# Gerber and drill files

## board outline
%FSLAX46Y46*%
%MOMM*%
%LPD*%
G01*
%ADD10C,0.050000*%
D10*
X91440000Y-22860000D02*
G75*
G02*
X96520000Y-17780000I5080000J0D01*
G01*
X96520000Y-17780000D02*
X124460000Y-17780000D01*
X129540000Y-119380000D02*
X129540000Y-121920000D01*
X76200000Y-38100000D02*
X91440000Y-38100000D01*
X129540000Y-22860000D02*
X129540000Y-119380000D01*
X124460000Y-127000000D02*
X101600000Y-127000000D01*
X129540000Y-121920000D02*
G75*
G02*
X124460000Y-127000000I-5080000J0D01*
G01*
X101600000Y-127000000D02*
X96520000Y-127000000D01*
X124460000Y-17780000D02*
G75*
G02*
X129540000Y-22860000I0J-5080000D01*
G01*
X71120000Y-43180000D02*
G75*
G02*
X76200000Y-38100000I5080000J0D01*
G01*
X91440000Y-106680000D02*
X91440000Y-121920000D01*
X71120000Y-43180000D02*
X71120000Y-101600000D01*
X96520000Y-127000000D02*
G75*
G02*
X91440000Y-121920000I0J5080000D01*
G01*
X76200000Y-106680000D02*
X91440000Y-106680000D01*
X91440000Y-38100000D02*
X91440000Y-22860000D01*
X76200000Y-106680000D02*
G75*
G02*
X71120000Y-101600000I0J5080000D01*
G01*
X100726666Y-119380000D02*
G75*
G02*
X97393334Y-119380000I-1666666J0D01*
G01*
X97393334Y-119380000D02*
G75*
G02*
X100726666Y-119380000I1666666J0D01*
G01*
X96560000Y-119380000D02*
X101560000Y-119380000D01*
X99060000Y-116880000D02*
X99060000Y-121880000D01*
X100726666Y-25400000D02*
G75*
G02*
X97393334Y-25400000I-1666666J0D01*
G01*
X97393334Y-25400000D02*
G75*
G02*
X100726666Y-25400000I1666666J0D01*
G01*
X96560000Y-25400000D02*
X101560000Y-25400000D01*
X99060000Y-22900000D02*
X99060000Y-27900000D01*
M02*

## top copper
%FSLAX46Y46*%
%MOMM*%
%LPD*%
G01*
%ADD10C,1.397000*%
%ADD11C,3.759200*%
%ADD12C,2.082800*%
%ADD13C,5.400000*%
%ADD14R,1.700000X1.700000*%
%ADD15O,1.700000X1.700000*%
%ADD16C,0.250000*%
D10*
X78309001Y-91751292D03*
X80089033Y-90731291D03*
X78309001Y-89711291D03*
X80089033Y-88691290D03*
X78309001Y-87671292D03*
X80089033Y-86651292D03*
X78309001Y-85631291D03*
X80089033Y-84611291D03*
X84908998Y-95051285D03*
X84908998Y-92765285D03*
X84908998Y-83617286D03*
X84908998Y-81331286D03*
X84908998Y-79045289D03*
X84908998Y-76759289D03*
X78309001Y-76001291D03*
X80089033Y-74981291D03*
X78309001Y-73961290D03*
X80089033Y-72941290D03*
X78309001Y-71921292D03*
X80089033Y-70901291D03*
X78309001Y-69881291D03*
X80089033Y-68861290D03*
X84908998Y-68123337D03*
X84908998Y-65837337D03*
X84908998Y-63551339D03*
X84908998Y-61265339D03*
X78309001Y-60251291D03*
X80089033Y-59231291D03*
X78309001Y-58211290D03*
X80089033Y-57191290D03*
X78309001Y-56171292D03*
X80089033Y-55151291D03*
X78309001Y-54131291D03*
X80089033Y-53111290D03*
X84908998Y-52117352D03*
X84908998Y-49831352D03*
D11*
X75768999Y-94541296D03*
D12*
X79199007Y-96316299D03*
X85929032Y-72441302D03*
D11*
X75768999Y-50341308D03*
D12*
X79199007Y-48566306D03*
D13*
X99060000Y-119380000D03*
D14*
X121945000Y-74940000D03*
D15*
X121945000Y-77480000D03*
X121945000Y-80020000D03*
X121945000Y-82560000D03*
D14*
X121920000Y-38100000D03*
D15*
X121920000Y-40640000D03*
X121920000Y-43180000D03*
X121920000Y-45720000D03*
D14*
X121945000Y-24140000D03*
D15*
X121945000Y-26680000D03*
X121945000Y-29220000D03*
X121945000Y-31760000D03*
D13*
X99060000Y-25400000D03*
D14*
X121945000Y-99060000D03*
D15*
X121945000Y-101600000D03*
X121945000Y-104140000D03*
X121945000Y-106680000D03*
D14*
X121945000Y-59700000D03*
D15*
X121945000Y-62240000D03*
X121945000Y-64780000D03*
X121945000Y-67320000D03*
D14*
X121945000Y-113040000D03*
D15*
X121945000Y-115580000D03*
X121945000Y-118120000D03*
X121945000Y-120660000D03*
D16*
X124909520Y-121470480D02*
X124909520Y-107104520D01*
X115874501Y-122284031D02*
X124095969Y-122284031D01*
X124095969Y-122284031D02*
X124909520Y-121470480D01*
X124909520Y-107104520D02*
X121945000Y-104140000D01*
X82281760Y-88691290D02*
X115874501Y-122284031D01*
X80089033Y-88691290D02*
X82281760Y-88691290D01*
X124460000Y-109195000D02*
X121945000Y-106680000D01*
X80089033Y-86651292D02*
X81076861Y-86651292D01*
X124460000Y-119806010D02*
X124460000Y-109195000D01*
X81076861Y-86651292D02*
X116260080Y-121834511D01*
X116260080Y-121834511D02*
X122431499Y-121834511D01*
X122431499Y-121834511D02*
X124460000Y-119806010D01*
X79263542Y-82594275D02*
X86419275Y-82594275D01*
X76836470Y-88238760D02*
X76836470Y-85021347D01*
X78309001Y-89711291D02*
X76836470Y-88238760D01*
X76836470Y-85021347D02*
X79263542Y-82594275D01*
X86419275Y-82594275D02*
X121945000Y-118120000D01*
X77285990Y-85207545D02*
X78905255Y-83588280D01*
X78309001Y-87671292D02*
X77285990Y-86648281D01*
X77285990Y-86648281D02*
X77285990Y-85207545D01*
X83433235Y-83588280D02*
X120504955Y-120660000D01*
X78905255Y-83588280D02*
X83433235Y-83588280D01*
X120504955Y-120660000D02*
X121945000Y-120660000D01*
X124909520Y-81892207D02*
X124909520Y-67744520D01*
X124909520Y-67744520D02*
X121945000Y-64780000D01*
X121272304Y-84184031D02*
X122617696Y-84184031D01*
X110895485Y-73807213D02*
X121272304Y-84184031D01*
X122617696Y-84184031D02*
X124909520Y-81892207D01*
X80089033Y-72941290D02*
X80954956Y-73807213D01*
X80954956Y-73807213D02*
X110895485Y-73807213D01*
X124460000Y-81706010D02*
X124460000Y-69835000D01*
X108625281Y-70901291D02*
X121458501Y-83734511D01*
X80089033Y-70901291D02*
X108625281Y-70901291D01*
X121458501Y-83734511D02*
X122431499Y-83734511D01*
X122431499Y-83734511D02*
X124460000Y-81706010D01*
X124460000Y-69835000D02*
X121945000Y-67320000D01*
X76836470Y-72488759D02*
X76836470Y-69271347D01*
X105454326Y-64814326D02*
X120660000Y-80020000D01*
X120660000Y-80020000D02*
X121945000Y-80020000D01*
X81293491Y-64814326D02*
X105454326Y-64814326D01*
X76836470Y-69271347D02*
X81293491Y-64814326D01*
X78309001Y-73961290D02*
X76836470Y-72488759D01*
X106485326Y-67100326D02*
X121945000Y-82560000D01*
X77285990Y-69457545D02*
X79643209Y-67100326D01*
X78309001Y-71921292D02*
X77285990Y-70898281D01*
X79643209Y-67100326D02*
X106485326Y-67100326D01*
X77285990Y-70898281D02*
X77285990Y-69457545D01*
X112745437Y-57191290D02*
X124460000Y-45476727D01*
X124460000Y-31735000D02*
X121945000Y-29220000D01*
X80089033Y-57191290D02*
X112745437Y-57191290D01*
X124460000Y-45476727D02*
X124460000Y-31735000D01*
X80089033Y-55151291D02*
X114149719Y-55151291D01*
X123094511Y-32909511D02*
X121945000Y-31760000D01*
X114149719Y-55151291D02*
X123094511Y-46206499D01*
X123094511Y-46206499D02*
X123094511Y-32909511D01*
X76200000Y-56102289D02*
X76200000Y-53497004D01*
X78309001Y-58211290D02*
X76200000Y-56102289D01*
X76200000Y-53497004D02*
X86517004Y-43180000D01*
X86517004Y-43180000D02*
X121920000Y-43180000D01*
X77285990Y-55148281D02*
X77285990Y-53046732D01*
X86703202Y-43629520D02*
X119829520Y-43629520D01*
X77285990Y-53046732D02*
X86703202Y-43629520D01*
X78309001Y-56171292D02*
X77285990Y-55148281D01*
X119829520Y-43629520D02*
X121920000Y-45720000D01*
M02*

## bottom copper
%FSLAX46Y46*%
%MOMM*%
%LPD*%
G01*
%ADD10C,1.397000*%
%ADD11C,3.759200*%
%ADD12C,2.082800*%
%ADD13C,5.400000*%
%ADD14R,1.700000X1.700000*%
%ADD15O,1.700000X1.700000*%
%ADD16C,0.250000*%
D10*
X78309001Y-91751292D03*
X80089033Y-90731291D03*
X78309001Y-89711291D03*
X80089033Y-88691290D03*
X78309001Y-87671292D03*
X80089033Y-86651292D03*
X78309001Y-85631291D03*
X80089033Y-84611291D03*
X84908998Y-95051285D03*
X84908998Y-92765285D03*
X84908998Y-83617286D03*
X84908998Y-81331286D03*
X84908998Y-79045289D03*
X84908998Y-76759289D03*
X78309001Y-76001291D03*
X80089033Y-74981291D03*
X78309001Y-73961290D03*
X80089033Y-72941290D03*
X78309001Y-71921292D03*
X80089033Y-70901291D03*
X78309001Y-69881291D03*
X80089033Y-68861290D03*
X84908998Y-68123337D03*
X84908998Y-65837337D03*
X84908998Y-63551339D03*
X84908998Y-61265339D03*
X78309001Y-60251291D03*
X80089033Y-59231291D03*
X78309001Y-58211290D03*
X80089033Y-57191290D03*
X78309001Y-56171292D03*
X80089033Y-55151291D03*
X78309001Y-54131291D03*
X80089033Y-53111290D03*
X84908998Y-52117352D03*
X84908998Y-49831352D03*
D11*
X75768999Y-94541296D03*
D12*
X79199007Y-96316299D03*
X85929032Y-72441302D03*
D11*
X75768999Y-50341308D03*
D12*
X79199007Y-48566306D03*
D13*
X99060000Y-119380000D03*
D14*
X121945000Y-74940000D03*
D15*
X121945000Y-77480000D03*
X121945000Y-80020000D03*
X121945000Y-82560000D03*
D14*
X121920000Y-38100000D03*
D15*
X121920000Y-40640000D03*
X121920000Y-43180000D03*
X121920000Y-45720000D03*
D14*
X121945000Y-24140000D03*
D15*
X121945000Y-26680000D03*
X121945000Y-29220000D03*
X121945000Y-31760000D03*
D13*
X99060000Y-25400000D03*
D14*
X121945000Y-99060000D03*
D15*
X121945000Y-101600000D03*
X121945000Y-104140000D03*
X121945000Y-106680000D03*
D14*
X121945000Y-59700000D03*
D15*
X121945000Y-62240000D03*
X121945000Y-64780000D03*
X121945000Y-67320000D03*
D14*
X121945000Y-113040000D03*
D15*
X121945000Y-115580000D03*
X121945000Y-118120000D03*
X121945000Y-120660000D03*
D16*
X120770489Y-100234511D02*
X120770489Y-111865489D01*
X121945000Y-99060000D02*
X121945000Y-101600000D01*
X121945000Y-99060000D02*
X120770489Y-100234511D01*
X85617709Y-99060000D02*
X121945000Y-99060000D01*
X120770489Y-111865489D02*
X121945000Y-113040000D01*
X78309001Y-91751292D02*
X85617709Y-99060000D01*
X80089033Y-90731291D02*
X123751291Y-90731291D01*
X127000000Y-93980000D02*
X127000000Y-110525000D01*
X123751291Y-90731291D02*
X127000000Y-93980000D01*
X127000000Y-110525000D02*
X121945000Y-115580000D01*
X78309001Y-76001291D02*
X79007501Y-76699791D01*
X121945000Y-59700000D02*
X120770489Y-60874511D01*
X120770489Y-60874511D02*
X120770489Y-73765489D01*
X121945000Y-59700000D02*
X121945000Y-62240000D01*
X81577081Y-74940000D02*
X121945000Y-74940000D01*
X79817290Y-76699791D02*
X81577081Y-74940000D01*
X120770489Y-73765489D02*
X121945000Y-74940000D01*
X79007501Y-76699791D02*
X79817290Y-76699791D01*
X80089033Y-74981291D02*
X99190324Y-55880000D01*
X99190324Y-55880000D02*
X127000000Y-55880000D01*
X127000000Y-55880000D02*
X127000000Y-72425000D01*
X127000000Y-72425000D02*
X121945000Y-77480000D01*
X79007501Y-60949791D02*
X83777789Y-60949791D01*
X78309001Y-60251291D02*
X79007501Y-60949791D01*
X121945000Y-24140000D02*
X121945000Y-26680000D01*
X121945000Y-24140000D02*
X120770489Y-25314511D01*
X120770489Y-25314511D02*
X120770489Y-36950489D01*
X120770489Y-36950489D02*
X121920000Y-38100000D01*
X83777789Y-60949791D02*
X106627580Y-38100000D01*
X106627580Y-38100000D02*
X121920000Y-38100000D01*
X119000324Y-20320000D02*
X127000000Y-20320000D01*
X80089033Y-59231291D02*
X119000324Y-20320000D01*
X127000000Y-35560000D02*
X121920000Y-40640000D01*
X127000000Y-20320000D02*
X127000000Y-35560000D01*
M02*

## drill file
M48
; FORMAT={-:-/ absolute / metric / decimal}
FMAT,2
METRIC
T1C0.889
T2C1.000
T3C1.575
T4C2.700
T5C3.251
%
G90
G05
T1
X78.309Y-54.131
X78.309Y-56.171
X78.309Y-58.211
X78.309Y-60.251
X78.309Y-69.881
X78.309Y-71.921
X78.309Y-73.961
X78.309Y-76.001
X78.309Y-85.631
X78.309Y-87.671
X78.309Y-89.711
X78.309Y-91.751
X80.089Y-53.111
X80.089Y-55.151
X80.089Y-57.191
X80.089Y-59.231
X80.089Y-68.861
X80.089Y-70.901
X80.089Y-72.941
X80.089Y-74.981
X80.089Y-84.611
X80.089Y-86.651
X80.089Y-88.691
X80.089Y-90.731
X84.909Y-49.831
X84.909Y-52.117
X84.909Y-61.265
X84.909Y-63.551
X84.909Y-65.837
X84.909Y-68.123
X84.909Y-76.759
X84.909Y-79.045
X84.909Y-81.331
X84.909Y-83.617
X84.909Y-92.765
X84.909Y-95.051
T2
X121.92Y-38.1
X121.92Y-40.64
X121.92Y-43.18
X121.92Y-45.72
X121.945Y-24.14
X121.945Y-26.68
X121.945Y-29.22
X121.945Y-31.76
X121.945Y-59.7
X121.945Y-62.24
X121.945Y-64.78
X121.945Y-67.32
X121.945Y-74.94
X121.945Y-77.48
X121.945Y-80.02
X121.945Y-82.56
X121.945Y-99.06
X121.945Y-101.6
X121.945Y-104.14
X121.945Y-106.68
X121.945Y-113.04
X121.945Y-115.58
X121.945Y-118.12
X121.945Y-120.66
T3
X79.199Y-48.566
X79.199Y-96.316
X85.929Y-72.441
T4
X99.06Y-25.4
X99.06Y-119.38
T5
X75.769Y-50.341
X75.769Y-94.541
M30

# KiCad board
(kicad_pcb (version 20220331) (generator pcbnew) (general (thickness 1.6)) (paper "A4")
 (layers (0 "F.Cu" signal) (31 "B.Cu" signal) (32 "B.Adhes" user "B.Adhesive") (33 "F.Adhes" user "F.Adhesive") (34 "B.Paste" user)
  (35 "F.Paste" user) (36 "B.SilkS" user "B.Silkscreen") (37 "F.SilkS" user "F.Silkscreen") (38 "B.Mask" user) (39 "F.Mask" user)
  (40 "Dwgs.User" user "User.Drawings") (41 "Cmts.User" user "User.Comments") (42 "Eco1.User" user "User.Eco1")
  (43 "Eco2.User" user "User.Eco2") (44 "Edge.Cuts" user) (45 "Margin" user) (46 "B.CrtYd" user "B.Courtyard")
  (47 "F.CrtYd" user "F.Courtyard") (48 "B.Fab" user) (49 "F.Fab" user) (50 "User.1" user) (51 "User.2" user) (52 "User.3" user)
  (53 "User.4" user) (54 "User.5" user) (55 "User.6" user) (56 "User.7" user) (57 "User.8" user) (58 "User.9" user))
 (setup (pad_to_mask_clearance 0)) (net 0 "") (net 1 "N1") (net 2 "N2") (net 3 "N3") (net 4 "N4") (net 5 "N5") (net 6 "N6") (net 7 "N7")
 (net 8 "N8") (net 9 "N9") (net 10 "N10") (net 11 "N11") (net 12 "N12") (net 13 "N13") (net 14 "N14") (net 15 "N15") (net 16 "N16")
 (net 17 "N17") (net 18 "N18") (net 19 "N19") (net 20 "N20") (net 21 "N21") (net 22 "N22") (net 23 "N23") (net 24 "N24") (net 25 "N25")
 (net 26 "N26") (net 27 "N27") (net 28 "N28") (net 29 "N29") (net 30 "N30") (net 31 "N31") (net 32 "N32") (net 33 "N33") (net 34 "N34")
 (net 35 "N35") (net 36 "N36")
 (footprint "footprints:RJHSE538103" (layer "F.Cu") (at 78.309001 91.751291 90)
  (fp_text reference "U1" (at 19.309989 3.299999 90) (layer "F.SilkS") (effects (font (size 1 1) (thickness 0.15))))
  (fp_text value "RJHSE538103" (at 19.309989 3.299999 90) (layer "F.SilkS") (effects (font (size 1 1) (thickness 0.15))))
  (pad "1" thru_hole circle locked (at -0.000001 0 90) (size 1.397 1.397) (drill 0.889) (layers *.Cu *.Mask) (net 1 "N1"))
  (pad "2" thru_hole circle locked (at 1.02 1.780032 90) (size 1.397 1.397) (drill 0.889) (layers *.Cu *.Mask) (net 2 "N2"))
  (pad "3" thru_hole circle locked (at 2.04 0 90) (size 1.397 1.397) (drill 0.889) (layers *.Cu *.Mask) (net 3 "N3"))
  (pad "4" thru_hole circle locked (at 3.060001 1.780032 90) (size 1.397 1.397) (drill 0.889) (layers *.Cu *.Mask) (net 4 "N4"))
  (pad "5" thru_hole circle locked (at 4.079999 0 90) (size 1.397 1.397) (drill 0.889) (layers *.Cu *.Mask) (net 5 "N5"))
  (pad "6" thru_hole circle locked (at 5.099999 1.780032 90) (size 1.397 1.397) (drill 0.889) (layers *.Cu *.Mask) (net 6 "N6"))
  (pad "7" thru_hole circle locked (at 6.12 0 90) (size 1.397 1.397) (drill 0.889) (layers *.Cu *.Mask) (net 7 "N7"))
  (pad "8" thru_hole circle locked (at 7.14 1.780032 90) (size 1.397 1.397) (drill 0.889) (layers *.Cu *.Mask) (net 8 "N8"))
  (pad "9" thru_hole circle locked (at -3.299994 6.599997 90) (size 1.397 1.397) (drill 0.889) (layers *.Cu *.Mask) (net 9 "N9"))
  (pad "10" thru_hole circle locked (at -1.013994 6.599997 90) (size 1.397 1.397) (drill 0.889) (layers *.Cu *.Mask) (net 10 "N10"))
  (pad "11" thru_hole circle locked (at 8.134005 6.599997 90) (size 1.397 1.397) (drill 0.889) (layers *.Cu *.Mask) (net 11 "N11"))
  (pad "12" thru_hole circle locked (at 10.420005 6.599997 90) (size 1.397 1.397) (drill 0.889) (layers *.Cu *.Mask) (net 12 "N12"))
  (pad "13" thru_hole circle locked (at 12.706002 6.599997 90) (size 1.397 1.397) (drill 0.889) (layers *.Cu *.Mask) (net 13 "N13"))
  (pad "14" thru_hole circle locked (at 14.992002 6.599997 90) (size 1.397 1.397) (drill 0.889) (layers *.Cu *.Mask) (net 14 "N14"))
  (pad "15" thru_hole circle locked (at 15.75 0 90) (size 1.397 1.397) (drill 0.889) (layers *.Cu *.Mask) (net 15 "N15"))
  (pad "16" thru_hole circle locked (at 16.77 1.780032 90) (size 1.397 1.397) (drill 0.889) (layers *.Cu *.Mask) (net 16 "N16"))
  (pad "17" thru_hole circle locked (at 17.790001 0 90) (size 1.397 1.397) (drill 0.889) (layers *.Cu *.Mask) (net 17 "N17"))
  (pad "18" thru_hole circle locked (at 18.810001 1.780032 90) (size 1.397 1.397) (drill 0.889) (layers *.Cu *.Mask) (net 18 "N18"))
  (pad "19" thru_hole circle locked (at 19.829999 0 90) (size 1.397 1.397) (drill 0.889) (layers *.Cu *.Mask) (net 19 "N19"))
  (pad "20" thru_hole circle locked (at 20.85 1.780032 90) (size 1.397 1.397) (drill 0.889) (layers *.Cu *.Mask) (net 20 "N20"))
  (pad "21" thru_hole circle locked (at 21.87 0 90) (size 1.397 1.397) (drill 0.889) (layers *.Cu *.Mask) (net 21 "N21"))
  (pad "22" thru_hole circle locked (at 22.890001 1.780032 90) (size 1.397 1.397) (drill 0.889) (layers *.Cu *.Mask) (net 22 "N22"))
  (pad "23" thru_hole circle locked (at 23.627954 6.599997 90) (size 1.397 1.397) (drill 0.889) (layers *.Cu *.Mask) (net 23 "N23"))
  (pad "24" thru_hole circle locked (at 25.913954 6.599997 90) (size 1.397 1.397) (drill 0.889) (layers *.Cu *.Mask) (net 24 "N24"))
  (pad "25" thru_hole circle locked (at 28.199952 6.599997 90) (size 1.397 1.397) (drill 0.889) (layers *.Cu *.Mask) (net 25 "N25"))
  (pad "26" thru_hole circle locked (at 30.485952 6.599997 90) (size 1.397 1.397) (drill 0.889) (layers *.Cu *.Mask) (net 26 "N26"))
  (pad "27" thru_hole circle locked (at 31.5 0 90) (size 1.397 1.397) (drill 0.889) (layers *.Cu *.Mask) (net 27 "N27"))
  (pad "28" thru_hole circle locked (at 32.52 1.780032 90) (size 1.397 1.397) (drill 0.889) (layers *.Cu *.Mask) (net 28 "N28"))
  (pad "29" thru_hole circle locked (at 33.540001 0 90) (size 1.397 1.397) (drill 0.889) (layers *.Cu *.Mask) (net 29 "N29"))
  (pad "30" thru_hole circle locked (at 34.560001 1.780032 90) (size 1.397 1.397) (drill 0.889) (layers *.Cu *.Mask) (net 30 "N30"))
  (pad "31" thru_hole circle locked (at 35.579999 0 90) (size 1.397 1.397) (drill 0.889) (layers *.Cu *.Mask) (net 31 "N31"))
  (pad "32" thru_hole circle locked (at 36.6 1.780032 90) (size 1.397 1.397) (drill 0.889) (layers *.Cu *.Mask) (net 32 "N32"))
  (pad "33" thru_hole circle locked (at 37.62 0 90) (size 1.397 1.397) (drill 0.889) (layers *.Cu *.Mask) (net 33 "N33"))
  (pad "34" thru_hole circle locked (at 38.640001 1.780032 90) (size 1.397 1.397) (drill 0.889) (layers *.Cu *.Mask) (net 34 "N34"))
  (pad "35" thru_hole circle locked (at 39.633939 6.599997 90) (size 1.397 1.397) (drill 0.889) (layers *.Cu *.Mask) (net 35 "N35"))
  (pad "36" thru_hole circle locked (at 41.919939 6.599997 90) (size 1.397 1.397) (drill 0.889) (layers *.Cu *.Mask) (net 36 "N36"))
  (pad "37" thru_hole circle locked (at -2.790005 -2.540002 90) (size 3.7592 3.7592) (drill 3.2512) (layers *.Cu *.Mask))
  (pad "38" thru_hole circle locked (at -4.565008 0.890006 90) (size 2.0828 2.0828) (drill 1.5748) (layers *.Cu *.Mask))
  (pad "39" thru_hole circle locked (at 19.309989 7.620031 90) (size 2.0828 2.0828) (drill 1.5748) (layers *.Cu *.Mask))
  (pad "40" thru_hole circle locked (at 41.409983 -2.540002 90) (size 3.7592 3.7592) (drill 3.2512) (layers *.Cu *.Mask))
  (pad "41" thru_hole circle locked (at 43.184985 0.890006 90) (size 2.0828 2.0828) (drill 1.5748) (layers *.Cu *.Mask)))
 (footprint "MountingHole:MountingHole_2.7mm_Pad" (layer "F.Cu") (at 99.06 119.38)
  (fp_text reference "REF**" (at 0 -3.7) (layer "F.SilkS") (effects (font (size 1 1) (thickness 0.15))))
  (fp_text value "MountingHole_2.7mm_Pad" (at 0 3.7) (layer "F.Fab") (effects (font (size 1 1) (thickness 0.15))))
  (pad "1" thru_hole circle (at 0 0) (size 5.4 5.4) (drill 2.7) (layers *.Cu *.Mask)))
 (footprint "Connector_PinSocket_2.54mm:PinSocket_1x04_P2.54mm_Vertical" (layer "F.Cu") (at 121.945 74.94)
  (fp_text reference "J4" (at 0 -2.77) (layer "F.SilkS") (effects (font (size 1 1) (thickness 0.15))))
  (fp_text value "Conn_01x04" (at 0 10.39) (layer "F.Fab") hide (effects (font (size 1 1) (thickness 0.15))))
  (pad "1" thru_hole rect (at 0 0) (size 1.7 1.7) (drill 1) (layers *.Cu *.Mask) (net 15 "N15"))
  (pad "2" thru_hole oval (at 0 2.54) (size 1.7 1.7) (drill 1) (layers *.Cu *.Mask) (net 16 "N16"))
  (pad "3" thru_hole oval (at 0 5.08) (size 1.7 1.7) (drill 1) (layers *.Cu *.Mask) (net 17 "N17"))
  (pad "4" thru_hole oval (at 0 7.62) (size 1.7 1.7) (drill 1) (layers *.Cu *.Mask) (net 19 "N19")))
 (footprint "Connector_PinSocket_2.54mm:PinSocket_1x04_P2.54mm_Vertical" (layer "F.Cu") (at 121.92 38.1)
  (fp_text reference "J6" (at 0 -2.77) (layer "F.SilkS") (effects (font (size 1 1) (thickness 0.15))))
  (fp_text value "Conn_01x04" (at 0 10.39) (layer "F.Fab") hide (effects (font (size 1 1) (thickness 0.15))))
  (pad "1" thru_hole rect (at 0 0) (size 1.7 1.7) (drill 1) (layers *.Cu *.Mask) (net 27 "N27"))
  (pad "2" thru_hole oval (at 0 2.54) (size 1.7 1.7) (drill 1) (layers *.Cu *.Mask) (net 28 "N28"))
  (pad "3" thru_hole oval (at 0 5.08) (size 1.7 1.7) (drill 1) (layers *.Cu *.Mask) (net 29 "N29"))
  (pad "4" thru_hole oval (at 0 7.62) (size 1.7 1.7) (drill 1) (layers *.Cu *.Mask) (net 31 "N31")))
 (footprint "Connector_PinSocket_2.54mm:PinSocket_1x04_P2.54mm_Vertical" (layer "F.Cu") (at 121.945 24.14)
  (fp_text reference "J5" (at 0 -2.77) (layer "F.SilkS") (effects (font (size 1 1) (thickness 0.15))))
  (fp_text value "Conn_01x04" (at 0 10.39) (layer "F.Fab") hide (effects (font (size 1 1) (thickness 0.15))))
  (pad "1" thru_hole rect (at 0 0) (size 1.7 1.7) (drill 1) (layers *.Cu *.Mask) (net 27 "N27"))
  (pad "2" thru_hole oval (at 0 2.54) (size 1.7 1.7) (drill 1) (layers *.Cu *.Mask) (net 27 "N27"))
  (pad "3" thru_hole oval (at 0 5.08) (size 1.7 1.7) (drill 1) (layers *.Cu *.Mask) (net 30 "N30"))
  (pad "4" thru_hole oval (at 0 7.62) (size 1.7 1.7) (drill 1) (layers *.Cu *.Mask) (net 32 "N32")))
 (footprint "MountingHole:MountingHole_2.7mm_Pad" (layer "F.Cu") (at 99.06 25.4)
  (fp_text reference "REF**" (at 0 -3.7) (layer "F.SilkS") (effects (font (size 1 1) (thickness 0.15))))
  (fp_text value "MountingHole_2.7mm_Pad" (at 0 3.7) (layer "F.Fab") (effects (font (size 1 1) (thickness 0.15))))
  (pad "1" thru_hole circle (at 0 0) (size 5.4 5.4) (drill 2.7) (layers *.Cu *.Mask)))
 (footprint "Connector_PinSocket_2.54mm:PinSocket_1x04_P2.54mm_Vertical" (layer "F.Cu") (at 121.945 99.06)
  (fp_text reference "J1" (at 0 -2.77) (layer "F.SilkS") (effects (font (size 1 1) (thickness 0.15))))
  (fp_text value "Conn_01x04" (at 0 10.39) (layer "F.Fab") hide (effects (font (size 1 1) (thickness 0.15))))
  (pad "1" thru_hole rect (at 0 0) (size 1.7 1.7) (drill 1) (layers *.Cu *.Mask) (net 1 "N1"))
  (pad "2" thru_hole oval (at 0 2.54) (size 1.7 1.7) (drill 1) (layers *.Cu *.Mask) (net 1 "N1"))
  (pad "3" thru_hole oval (at 0 5.08) (size 1.7 1.7) (drill 1) (layers *.Cu *.Mask) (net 4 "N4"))
  (pad "4" thru_hole oval (at 0 7.62) (size 1.7 1.7) (drill 1) (layers *.Cu *.Mask) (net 6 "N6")))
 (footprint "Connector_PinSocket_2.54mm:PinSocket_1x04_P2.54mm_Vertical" (layer "F.Cu") (at 121.945 59.7)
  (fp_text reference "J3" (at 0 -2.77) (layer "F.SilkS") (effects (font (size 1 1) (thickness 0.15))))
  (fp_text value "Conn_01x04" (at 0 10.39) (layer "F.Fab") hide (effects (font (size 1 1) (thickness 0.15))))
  (pad "1" thru_hole rect (at 0 0) (size 1.7 1.7) (drill 1) (layers *.Cu *.Mask) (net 15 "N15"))
  (pad "2" thru_hole oval (at 0 2.54) (size 1.7 1.7) (drill 1) (layers *.Cu *.Mask) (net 15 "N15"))
  (pad "3" thru_hole oval (at 0 5.08) (size 1.7 1.7) (drill 1) (layers *.Cu *.Mask) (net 18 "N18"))
  (pad "4" thru_hole oval (at 0 7.62) (size 1.7 1.7) (drill 1) (layers *.Cu *.Mask) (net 20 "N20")))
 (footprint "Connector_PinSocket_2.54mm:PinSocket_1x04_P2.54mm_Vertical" (layer "F.Cu") (at 121.945 113.04)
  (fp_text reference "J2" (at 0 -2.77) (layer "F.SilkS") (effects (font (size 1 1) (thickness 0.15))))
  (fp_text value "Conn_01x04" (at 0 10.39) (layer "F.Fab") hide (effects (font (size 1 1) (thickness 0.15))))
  (pad "1" thru_hole rect (at 0 0) (size 1.7 1.7) (drill 1) (layers *.Cu *.Mask) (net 1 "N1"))
  (pad "2" thru_hole oval (at 0 2.54) (size 1.7 1.7) (drill 1) (layers *.Cu *.Mask) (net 2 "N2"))
  (pad "3" thru_hole oval (at 0 5.08) (size 1.7 1.7) (drill 1) (layers *.Cu *.Mask) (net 3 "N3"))
  (pad "4" thru_hole oval (at 0 7.62) (size 1.7 1.7) (drill 1) (layers *.Cu *.Mask) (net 5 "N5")))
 (gr_arc (start 91.44 22.86) (mid 92.927898 19.267898) (end 96.52 17.78) (stroke (width 0.05) (type default)) (layer "Edge.Cuts"))
 (gr_line (start 96.52 17.78) (end 124.46 17.78) (stroke (width 0.05) (type default)) (layer "Edge.Cuts"))
 (gr_line (start 129.54 119.38) (end 129.54 121.92) (stroke (width 0.05) (type default)) (layer "Edge.Cuts"))
 (gr_line (start 76.2 38.1) (end 91.44 38.1) (stroke (width 0.05) (type default)) (layer "Edge.Cuts"))
 (gr_line (start 129.54 22.86) (end 129.54 119.38) (stroke (width 0.05) (type default)) (layer "Edge.Cuts"))
 (gr_line (start 124.46 127) (end 101.6 127) (stroke (width 0.05) (type default)) (layer "Edge.Cuts"))
 (gr_arc (start 129.54 121.92) (mid 128.052102 125.512102) (end 124.46 127) (stroke (width 0.05) (type default)) (layer "Edge.Cuts"))
 (gr_line (start 101.6 127) (end 96.52 127) (stroke (width 0.05) (type default)) (layer "Edge.Cuts"))
 (gr_arc (start 124.46 17.78) (mid 128.052102 19.267898) (end 129.54 22.86) (stroke (width 0.05) (type default)) (layer "Edge.Cuts"))
 (gr_arc (start 71.12 43.18) (mid 72.607898 39.587898) (end 76.2 38.1) (stroke (width 0.05) (type default)) (layer "Edge.Cuts"))
 (gr_line (start 91.44 106.68) (end 91.44 121.92) (stroke (width 0.05) (type default)) (layer "Edge.Cuts"))
 (gr_line (start 71.12 43.18) (end 71.12 101.6) (stroke (width 0.05) (type default)) (layer "Edge.Cuts"))
 (gr_arc (start 96.52 127) (mid 92.927898 125.512102) (end 91.44 121.92) (stroke (width 0.05) (type default)) (layer "Edge.Cuts"))
 (gr_line (start 76.2 106.68) (end 91.44 106.68) (stroke (width 0.05) (type default)) (layer "Edge.Cuts"))
 (gr_line (start 91.44 38.1) (end 91.44 22.86) (stroke (width 0.05) (type default)) (layer "Edge.Cuts"))
 (gr_arc (start 76.2 106.68) (mid 72.607898 105.192102) (end 71.12 101.6) (stroke (width 0.05) (type default)) (layer "Edge.Cuts"))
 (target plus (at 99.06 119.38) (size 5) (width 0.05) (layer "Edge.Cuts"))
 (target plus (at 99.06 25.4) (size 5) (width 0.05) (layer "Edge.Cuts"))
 (segment (start 120.770489 100.234511) (end 120.770489 111.865489) (width 0.25) (layer "B.Cu") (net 1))
 (segment (start 121.945 99.06) (end 121.945 101.6) (width 0.25) (layer "B.Cu") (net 1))
 (segment (start 121.945 99.06) (end 120.770489 100.234511) (width 0.25) (layer "B.Cu") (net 1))
 (segment (start 85.617709 99.06) (end 121.945 99.06) (width 0.25) (layer "B.Cu") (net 1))
 (segment (start 120.770489 111.865489) (end 121.945 113.04) (width 0.25) (layer "B.Cu") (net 1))
 (segment (start 78.309001 91.751292) (end 85.617709 99.06) (width 0.25) (layer "B.Cu") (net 1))
 (segment (start 124.90952 121.47048) (end 124.90952 107.10452) (width 0.25) (layer "F.Cu") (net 4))
 (segment (start 115.874501 122.284031) (end 124.095969 122.284031) (width 0.25) (layer "F.Cu") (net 4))
 (segment (start 124.095969 122.284031) (end 124.90952 121.47048) (width 0.25) (layer "F.Cu") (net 4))
 (segment (start 124.90952 107.10452) (end 121.945 104.14) (width 0.25) (layer "F.Cu") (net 4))
 (segment (start 82.28176 88.69129) (end 115.874501 122.284031) (width 0.25) (layer "F.Cu") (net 4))
 (segment (start 80.089033 88.69129) (end 82.28176 88.69129) (width 0.25) (layer "F.Cu") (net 4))
 (segment (start 124.46 109.195) (end 121.945 106.68) (width 0.25) (layer "F.Cu") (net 6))
 (segment (start 80.089033 86.651292) (end 81.076861 86.651292) (width 0.25) (layer "F.Cu") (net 6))
 (segment (start 124.46 119.80601) (end 124.46 109.195) (width 0.25) (layer "F.Cu") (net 6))
 (segment (start 81.076861 86.651292) (end 116.26008 121.834511) (width 0.25) (layer "F.Cu") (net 6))
 (segment (start 116.26008 121.834511) (end 122.431499 121.834511) (width 0.25) (layer "F.Cu") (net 6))
 (segment (start 122.431499 121.834511) (end 124.46 119.80601) (width 0.25) (layer "F.Cu") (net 6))
 (segment (start 80.089033 90.731291) (end 123.751291 90.731291) (width 0.25) (layer "B.Cu") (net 2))
 (segment (start 127 93.98) (end 127 110.525) (width 0.25) (layer "B.Cu") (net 2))
 (segment (start 123.751291 90.731291) (end 127 93.98) (width 0.25) (layer "B.Cu") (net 2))
 (segment (start 127 110.525) (end 121.945 115.58) (width 0.25) (layer "B.Cu") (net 2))
 (segment (start 79.263542 82.594275) (end 86.419275 82.594275) (width 0.25) (layer "F.Cu") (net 3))
 (segment (start 76.83647 88.23876) (end 76.83647 85.021347) (width 0.25) (layer "F.Cu") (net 3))
 (segment (start 78.309001 89.711291) (end 76.83647 88.23876) (width 0.25) (layer "F.Cu") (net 3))
 (segment (start 76.83647 85.021347) (end 79.263542 82.594275) (width 0.25) (layer "F.Cu") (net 3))
 (segment (start 86.419275 82.594275) (end 121.945 118.12) (width 0.25) (layer "F.Cu") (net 3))
 (segment (start 77.28599 85.207545) (end 78.905255 83.58828) (width 0.25) (layer "F.Cu") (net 5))
 (segment (start 78.309001 87.671292) (end 77.28599 86.648281) (width 0.25) (layer "F.Cu") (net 5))
 (segment (start 77.28599 86.648281) (end 77.28599 85.207545) (width 0.25) (layer "F.Cu") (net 5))
 (segment (start 83.433235 83.58828) (end 120.504955 120.66) (width 0.25) (layer "F.Cu") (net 5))
 (segment (start 78.905255 83.58828) (end 83.433235 83.58828) (width 0.25) (layer "F.Cu") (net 5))
 (segment (start 120.504955 120.66) (end 121.945 120.66) (width 0.25) (layer "F.Cu") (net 5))
 (segment (start 78.309001 76.001291) (end 79.007501 76.699791) (width 0.25) (layer "B.Cu") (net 15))
 (segment (start 121.945 59.7) (end 120.770489 60.874511) (width 0.25) (layer "B.Cu") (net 15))
 (segment (start 120.770489 60.874511) (end 120.770489 73.765489) (width 0.25) (layer "B.Cu") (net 15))
 (segment (start 121.945 59.7) (end 121.945 62.24) (width 0.25) (layer "B.Cu") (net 15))
 (segment (start 81.577081 74.94) (end 121.945 74.94) (width 0.25) (layer "B.Cu") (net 15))
 (segment (start 79.81729 76.699791) (end 81.577081 74.94) (width 0.25) (layer "B.Cu") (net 15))
 (segment (start 120.770489 73.765489) (end 121.945 74.94) (width 0.25) (layer "B.Cu") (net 15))
 (segment (start 79.007501 76.699791) (end 79.81729 76.699791) (width 0.25) (layer "B.Cu") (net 15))
 (segment (start 124.90952 81.892207) (end 124.90952 67.74452) (width 0.25) (layer "F.Cu") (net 18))
 (segment (start 124.90952 67.74452) (end 121.945 64.78) (width 0.25) (layer "F.Cu") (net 18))
 (segment (start 121.272304 84.184031) (end 122.617696 84.184031) (width 0.25) (layer "F.Cu") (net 18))
 (segment (start 110.895485 73.807213) (end 121.272304 84.184031) (width 0.25) (layer "F.Cu") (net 18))
 (segment (start 122.617696 84.184031) (end 124.90952 81.892207) (width 0.25) (layer "F.Cu") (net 18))
 (segment (start 80.089033 72.94129) (end 80.954956 73.807213) (width 0.25) (layer "F.Cu") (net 18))
 (segment (start 80.954956 73.807213) (end 110.895485 73.807213) (width 0.25) (layer "F.Cu") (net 18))
 (segment (start 124.46 81.70601) (end 124.46 69.835) (width 0.25) (layer "F.Cu") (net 20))
 (segment (start 108.625281 70.901291) (end 121.458501 83.734511) (width 0.25) (layer "F.Cu") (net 20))
 (segment (start 80.089033 70.901291) (end 108.625281 70.901291) (width 0.25) (layer "F.Cu") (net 20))
 (segment (start 121.458501 83.734511) (end 122.431499 83.734511) (width 0.25) (layer "F.Cu") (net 20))
 (segment (start 122.431499 83.734511) (end 124.46 81.70601) (width 0.25) (layer "F.Cu") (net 20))
 (segment (start 124.46 69.835) (end 121.945 67.32) (width 0.25) (layer "F.Cu") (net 20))
 (segment (start 80.089033 74.981291) (end 99.190324 55.88) (width 0.25) (layer "B.Cu") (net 16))
 (segment (start 99.190324 55.88) (end 127 55.88) (width 0.25) (layer "B.Cu") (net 16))
 (segment (start 127 55.88) (end 127 72.425) (width 0.25) (layer "B.Cu") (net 16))
 (segment (start 127 72.425) (end 121.945 77.48) (width 0.25) (layer "B.Cu") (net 16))
 (segment (start 76.83647 72.488759) (end 76.83647 69.271347) (width 0.25) (layer "F.Cu") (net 17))
 (segment (start 105.454326 64.814326) (end 120.66 80.02) (width 0.25) (layer "F.Cu") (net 17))
 (segment (start 120.66 80.02) (end 121.945 80.02) (width 0.25) (layer "F.Cu") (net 17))
 (segment (start 81.293491 64.814326) (end 105.454326 64.814326) (width 0.25) (layer "F.Cu") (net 17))
 (segment (start 76.83647 69.271347) (end 81.293491 64.814326) (width 0.25) (layer "F.Cu") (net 17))
 (segment (start 78.309001 73.96129) (end 76.83647 72.488759) (width 0.25) (layer "F.Cu") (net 17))
 (segment (start 106.485326 67.100326) (end 121.945 82.56) (width 0.25) (layer "F.Cu") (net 19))
 (segment (start 77.28599 69.457545) (end 79.643209 67.100326) (width 0.25) (layer "F.Cu") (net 19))
 (segment (start 78.309001 71.921292) (end 77.28599 70.898281) (width 0.25) (layer "F.Cu") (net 19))
 (segment (start 79.643209 67.100326) (end 106.485326 67.100326) (width 0.25) (layer "F.Cu") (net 19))
 (segment (start 77.28599 70.898281) (end 77.28599 69.457545) (width 0.25) (layer "F.Cu") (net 19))
 (segment (start 79.007501 60.949791) (end 83.777789 60.949791) (width 0.25) (layer "B.Cu") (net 27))
 (segment (start 78.309001 60.251291) (end 79.007501 60.949791) (width 0.25) (layer "B.Cu") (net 27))
 (segment (start 121.945 24.14) (end 121.945 26.68) (width 0.25) (layer "B.Cu") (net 27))
 (segment (start 121.945 24.14) (end 120.770489 25.314511) (width 0.25) (layer "B.Cu") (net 27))
 (segment (start 120.770489 25.314511) (end 120.770489 36.950489) (width 0.25) (layer "B.Cu") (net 27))
 (segment (start 120.770489 36.950489) (end 121.92 38.1) (width 0.25) (layer "B.Cu") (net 27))
 (segment (start 83.777789 60.949791) (end 106.62758 38.1) (width 0.25) (layer "B.Cu") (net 27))
 (segment (start 106.62758 38.1) (end 121.92 38.1) (width 0.25) (layer "B.Cu") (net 27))
 (segment (start 112.745437 57.19129) (end 124.46 45.476727) (width 0.25) (layer "F.Cu") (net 30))
 (segment (start 124.46 31.735) (end 121.945 29.22) (width 0.25) (layer "F.Cu") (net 30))
 (segment (start 80.089033 57.19129) (end 112.745437 57.19129) (width 0.25) (layer "F.Cu") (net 30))
 (segment (start 124.46 45.476727) (end 124.46 31.735) (width 0.25) (layer "F.Cu") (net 30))
 (segment (start 80.089033 55.151291) (end 114.149719 55.151291) (width 0.25) (layer "F.Cu") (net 32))
 (segment (start 123.094511 32.909511) (end 121.945 31.76) (width 0.25) (layer "F.Cu") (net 32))
 (segment (start 114.149719 55.151291) (end 123.094511 46.206499) (width 0.25) (layer "F.Cu") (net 32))
 (segment (start 123.094511 46.206499) (end 123.094511 32.909511) (width 0.25) (layer "F.Cu") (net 32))
 (segment (start 119.000324 20.32) (end 127 20.32) (width 0.25) (layer "B.Cu") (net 28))
 (segment (start 80.089033 59.231291) (end 119.000324 20.32) (width 0.25) (layer "B.Cu") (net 28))
 (segment (start 127 35.56) (end 121.92 40.64) (width 0.25) (layer "B.Cu") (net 28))
 (segment (start 127 20.32) (end 127 35.56) (width 0.25) (layer "B.Cu") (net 28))
 (segment (start 76.2 56.102289) (end 76.2 53.497004) (width 0.25) (layer "F.Cu") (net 29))
 (segment (start 78.309001 58.21129) (end 76.2 56.102289) (width 0.25) (layer "F.Cu") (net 29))
 (segment (start 76.2 53.497004) (end 86.517004 43.18) (width 0.25) (layer "F.Cu") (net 29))
 (segment (start 86.517004 43.18) (end 121.92 43.18) (width 0.25) (layer "F.Cu") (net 29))
 (segment (start 77.28599 55.148281) (end 77.28599 53.046732) (width 0.25) (layer "F.Cu") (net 31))
 (segment (start 86.703202 43.62952) (end 119.82952 43.62952) (width 0.25) (layer "F.Cu") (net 31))
 (segment (start 77.28599 53.046732) (end 86.703202 43.62952) (width 0.25) (layer "F.Cu") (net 31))
 (segment (start 78.309001 56.171292) (end 77.28599 55.148281) (width 0.25) (layer "F.Cu") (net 31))
 (segment (start 119.82952 43.62952) (end 121.92 45.72) (width 0.25) (layer "F.Cu") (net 31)))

